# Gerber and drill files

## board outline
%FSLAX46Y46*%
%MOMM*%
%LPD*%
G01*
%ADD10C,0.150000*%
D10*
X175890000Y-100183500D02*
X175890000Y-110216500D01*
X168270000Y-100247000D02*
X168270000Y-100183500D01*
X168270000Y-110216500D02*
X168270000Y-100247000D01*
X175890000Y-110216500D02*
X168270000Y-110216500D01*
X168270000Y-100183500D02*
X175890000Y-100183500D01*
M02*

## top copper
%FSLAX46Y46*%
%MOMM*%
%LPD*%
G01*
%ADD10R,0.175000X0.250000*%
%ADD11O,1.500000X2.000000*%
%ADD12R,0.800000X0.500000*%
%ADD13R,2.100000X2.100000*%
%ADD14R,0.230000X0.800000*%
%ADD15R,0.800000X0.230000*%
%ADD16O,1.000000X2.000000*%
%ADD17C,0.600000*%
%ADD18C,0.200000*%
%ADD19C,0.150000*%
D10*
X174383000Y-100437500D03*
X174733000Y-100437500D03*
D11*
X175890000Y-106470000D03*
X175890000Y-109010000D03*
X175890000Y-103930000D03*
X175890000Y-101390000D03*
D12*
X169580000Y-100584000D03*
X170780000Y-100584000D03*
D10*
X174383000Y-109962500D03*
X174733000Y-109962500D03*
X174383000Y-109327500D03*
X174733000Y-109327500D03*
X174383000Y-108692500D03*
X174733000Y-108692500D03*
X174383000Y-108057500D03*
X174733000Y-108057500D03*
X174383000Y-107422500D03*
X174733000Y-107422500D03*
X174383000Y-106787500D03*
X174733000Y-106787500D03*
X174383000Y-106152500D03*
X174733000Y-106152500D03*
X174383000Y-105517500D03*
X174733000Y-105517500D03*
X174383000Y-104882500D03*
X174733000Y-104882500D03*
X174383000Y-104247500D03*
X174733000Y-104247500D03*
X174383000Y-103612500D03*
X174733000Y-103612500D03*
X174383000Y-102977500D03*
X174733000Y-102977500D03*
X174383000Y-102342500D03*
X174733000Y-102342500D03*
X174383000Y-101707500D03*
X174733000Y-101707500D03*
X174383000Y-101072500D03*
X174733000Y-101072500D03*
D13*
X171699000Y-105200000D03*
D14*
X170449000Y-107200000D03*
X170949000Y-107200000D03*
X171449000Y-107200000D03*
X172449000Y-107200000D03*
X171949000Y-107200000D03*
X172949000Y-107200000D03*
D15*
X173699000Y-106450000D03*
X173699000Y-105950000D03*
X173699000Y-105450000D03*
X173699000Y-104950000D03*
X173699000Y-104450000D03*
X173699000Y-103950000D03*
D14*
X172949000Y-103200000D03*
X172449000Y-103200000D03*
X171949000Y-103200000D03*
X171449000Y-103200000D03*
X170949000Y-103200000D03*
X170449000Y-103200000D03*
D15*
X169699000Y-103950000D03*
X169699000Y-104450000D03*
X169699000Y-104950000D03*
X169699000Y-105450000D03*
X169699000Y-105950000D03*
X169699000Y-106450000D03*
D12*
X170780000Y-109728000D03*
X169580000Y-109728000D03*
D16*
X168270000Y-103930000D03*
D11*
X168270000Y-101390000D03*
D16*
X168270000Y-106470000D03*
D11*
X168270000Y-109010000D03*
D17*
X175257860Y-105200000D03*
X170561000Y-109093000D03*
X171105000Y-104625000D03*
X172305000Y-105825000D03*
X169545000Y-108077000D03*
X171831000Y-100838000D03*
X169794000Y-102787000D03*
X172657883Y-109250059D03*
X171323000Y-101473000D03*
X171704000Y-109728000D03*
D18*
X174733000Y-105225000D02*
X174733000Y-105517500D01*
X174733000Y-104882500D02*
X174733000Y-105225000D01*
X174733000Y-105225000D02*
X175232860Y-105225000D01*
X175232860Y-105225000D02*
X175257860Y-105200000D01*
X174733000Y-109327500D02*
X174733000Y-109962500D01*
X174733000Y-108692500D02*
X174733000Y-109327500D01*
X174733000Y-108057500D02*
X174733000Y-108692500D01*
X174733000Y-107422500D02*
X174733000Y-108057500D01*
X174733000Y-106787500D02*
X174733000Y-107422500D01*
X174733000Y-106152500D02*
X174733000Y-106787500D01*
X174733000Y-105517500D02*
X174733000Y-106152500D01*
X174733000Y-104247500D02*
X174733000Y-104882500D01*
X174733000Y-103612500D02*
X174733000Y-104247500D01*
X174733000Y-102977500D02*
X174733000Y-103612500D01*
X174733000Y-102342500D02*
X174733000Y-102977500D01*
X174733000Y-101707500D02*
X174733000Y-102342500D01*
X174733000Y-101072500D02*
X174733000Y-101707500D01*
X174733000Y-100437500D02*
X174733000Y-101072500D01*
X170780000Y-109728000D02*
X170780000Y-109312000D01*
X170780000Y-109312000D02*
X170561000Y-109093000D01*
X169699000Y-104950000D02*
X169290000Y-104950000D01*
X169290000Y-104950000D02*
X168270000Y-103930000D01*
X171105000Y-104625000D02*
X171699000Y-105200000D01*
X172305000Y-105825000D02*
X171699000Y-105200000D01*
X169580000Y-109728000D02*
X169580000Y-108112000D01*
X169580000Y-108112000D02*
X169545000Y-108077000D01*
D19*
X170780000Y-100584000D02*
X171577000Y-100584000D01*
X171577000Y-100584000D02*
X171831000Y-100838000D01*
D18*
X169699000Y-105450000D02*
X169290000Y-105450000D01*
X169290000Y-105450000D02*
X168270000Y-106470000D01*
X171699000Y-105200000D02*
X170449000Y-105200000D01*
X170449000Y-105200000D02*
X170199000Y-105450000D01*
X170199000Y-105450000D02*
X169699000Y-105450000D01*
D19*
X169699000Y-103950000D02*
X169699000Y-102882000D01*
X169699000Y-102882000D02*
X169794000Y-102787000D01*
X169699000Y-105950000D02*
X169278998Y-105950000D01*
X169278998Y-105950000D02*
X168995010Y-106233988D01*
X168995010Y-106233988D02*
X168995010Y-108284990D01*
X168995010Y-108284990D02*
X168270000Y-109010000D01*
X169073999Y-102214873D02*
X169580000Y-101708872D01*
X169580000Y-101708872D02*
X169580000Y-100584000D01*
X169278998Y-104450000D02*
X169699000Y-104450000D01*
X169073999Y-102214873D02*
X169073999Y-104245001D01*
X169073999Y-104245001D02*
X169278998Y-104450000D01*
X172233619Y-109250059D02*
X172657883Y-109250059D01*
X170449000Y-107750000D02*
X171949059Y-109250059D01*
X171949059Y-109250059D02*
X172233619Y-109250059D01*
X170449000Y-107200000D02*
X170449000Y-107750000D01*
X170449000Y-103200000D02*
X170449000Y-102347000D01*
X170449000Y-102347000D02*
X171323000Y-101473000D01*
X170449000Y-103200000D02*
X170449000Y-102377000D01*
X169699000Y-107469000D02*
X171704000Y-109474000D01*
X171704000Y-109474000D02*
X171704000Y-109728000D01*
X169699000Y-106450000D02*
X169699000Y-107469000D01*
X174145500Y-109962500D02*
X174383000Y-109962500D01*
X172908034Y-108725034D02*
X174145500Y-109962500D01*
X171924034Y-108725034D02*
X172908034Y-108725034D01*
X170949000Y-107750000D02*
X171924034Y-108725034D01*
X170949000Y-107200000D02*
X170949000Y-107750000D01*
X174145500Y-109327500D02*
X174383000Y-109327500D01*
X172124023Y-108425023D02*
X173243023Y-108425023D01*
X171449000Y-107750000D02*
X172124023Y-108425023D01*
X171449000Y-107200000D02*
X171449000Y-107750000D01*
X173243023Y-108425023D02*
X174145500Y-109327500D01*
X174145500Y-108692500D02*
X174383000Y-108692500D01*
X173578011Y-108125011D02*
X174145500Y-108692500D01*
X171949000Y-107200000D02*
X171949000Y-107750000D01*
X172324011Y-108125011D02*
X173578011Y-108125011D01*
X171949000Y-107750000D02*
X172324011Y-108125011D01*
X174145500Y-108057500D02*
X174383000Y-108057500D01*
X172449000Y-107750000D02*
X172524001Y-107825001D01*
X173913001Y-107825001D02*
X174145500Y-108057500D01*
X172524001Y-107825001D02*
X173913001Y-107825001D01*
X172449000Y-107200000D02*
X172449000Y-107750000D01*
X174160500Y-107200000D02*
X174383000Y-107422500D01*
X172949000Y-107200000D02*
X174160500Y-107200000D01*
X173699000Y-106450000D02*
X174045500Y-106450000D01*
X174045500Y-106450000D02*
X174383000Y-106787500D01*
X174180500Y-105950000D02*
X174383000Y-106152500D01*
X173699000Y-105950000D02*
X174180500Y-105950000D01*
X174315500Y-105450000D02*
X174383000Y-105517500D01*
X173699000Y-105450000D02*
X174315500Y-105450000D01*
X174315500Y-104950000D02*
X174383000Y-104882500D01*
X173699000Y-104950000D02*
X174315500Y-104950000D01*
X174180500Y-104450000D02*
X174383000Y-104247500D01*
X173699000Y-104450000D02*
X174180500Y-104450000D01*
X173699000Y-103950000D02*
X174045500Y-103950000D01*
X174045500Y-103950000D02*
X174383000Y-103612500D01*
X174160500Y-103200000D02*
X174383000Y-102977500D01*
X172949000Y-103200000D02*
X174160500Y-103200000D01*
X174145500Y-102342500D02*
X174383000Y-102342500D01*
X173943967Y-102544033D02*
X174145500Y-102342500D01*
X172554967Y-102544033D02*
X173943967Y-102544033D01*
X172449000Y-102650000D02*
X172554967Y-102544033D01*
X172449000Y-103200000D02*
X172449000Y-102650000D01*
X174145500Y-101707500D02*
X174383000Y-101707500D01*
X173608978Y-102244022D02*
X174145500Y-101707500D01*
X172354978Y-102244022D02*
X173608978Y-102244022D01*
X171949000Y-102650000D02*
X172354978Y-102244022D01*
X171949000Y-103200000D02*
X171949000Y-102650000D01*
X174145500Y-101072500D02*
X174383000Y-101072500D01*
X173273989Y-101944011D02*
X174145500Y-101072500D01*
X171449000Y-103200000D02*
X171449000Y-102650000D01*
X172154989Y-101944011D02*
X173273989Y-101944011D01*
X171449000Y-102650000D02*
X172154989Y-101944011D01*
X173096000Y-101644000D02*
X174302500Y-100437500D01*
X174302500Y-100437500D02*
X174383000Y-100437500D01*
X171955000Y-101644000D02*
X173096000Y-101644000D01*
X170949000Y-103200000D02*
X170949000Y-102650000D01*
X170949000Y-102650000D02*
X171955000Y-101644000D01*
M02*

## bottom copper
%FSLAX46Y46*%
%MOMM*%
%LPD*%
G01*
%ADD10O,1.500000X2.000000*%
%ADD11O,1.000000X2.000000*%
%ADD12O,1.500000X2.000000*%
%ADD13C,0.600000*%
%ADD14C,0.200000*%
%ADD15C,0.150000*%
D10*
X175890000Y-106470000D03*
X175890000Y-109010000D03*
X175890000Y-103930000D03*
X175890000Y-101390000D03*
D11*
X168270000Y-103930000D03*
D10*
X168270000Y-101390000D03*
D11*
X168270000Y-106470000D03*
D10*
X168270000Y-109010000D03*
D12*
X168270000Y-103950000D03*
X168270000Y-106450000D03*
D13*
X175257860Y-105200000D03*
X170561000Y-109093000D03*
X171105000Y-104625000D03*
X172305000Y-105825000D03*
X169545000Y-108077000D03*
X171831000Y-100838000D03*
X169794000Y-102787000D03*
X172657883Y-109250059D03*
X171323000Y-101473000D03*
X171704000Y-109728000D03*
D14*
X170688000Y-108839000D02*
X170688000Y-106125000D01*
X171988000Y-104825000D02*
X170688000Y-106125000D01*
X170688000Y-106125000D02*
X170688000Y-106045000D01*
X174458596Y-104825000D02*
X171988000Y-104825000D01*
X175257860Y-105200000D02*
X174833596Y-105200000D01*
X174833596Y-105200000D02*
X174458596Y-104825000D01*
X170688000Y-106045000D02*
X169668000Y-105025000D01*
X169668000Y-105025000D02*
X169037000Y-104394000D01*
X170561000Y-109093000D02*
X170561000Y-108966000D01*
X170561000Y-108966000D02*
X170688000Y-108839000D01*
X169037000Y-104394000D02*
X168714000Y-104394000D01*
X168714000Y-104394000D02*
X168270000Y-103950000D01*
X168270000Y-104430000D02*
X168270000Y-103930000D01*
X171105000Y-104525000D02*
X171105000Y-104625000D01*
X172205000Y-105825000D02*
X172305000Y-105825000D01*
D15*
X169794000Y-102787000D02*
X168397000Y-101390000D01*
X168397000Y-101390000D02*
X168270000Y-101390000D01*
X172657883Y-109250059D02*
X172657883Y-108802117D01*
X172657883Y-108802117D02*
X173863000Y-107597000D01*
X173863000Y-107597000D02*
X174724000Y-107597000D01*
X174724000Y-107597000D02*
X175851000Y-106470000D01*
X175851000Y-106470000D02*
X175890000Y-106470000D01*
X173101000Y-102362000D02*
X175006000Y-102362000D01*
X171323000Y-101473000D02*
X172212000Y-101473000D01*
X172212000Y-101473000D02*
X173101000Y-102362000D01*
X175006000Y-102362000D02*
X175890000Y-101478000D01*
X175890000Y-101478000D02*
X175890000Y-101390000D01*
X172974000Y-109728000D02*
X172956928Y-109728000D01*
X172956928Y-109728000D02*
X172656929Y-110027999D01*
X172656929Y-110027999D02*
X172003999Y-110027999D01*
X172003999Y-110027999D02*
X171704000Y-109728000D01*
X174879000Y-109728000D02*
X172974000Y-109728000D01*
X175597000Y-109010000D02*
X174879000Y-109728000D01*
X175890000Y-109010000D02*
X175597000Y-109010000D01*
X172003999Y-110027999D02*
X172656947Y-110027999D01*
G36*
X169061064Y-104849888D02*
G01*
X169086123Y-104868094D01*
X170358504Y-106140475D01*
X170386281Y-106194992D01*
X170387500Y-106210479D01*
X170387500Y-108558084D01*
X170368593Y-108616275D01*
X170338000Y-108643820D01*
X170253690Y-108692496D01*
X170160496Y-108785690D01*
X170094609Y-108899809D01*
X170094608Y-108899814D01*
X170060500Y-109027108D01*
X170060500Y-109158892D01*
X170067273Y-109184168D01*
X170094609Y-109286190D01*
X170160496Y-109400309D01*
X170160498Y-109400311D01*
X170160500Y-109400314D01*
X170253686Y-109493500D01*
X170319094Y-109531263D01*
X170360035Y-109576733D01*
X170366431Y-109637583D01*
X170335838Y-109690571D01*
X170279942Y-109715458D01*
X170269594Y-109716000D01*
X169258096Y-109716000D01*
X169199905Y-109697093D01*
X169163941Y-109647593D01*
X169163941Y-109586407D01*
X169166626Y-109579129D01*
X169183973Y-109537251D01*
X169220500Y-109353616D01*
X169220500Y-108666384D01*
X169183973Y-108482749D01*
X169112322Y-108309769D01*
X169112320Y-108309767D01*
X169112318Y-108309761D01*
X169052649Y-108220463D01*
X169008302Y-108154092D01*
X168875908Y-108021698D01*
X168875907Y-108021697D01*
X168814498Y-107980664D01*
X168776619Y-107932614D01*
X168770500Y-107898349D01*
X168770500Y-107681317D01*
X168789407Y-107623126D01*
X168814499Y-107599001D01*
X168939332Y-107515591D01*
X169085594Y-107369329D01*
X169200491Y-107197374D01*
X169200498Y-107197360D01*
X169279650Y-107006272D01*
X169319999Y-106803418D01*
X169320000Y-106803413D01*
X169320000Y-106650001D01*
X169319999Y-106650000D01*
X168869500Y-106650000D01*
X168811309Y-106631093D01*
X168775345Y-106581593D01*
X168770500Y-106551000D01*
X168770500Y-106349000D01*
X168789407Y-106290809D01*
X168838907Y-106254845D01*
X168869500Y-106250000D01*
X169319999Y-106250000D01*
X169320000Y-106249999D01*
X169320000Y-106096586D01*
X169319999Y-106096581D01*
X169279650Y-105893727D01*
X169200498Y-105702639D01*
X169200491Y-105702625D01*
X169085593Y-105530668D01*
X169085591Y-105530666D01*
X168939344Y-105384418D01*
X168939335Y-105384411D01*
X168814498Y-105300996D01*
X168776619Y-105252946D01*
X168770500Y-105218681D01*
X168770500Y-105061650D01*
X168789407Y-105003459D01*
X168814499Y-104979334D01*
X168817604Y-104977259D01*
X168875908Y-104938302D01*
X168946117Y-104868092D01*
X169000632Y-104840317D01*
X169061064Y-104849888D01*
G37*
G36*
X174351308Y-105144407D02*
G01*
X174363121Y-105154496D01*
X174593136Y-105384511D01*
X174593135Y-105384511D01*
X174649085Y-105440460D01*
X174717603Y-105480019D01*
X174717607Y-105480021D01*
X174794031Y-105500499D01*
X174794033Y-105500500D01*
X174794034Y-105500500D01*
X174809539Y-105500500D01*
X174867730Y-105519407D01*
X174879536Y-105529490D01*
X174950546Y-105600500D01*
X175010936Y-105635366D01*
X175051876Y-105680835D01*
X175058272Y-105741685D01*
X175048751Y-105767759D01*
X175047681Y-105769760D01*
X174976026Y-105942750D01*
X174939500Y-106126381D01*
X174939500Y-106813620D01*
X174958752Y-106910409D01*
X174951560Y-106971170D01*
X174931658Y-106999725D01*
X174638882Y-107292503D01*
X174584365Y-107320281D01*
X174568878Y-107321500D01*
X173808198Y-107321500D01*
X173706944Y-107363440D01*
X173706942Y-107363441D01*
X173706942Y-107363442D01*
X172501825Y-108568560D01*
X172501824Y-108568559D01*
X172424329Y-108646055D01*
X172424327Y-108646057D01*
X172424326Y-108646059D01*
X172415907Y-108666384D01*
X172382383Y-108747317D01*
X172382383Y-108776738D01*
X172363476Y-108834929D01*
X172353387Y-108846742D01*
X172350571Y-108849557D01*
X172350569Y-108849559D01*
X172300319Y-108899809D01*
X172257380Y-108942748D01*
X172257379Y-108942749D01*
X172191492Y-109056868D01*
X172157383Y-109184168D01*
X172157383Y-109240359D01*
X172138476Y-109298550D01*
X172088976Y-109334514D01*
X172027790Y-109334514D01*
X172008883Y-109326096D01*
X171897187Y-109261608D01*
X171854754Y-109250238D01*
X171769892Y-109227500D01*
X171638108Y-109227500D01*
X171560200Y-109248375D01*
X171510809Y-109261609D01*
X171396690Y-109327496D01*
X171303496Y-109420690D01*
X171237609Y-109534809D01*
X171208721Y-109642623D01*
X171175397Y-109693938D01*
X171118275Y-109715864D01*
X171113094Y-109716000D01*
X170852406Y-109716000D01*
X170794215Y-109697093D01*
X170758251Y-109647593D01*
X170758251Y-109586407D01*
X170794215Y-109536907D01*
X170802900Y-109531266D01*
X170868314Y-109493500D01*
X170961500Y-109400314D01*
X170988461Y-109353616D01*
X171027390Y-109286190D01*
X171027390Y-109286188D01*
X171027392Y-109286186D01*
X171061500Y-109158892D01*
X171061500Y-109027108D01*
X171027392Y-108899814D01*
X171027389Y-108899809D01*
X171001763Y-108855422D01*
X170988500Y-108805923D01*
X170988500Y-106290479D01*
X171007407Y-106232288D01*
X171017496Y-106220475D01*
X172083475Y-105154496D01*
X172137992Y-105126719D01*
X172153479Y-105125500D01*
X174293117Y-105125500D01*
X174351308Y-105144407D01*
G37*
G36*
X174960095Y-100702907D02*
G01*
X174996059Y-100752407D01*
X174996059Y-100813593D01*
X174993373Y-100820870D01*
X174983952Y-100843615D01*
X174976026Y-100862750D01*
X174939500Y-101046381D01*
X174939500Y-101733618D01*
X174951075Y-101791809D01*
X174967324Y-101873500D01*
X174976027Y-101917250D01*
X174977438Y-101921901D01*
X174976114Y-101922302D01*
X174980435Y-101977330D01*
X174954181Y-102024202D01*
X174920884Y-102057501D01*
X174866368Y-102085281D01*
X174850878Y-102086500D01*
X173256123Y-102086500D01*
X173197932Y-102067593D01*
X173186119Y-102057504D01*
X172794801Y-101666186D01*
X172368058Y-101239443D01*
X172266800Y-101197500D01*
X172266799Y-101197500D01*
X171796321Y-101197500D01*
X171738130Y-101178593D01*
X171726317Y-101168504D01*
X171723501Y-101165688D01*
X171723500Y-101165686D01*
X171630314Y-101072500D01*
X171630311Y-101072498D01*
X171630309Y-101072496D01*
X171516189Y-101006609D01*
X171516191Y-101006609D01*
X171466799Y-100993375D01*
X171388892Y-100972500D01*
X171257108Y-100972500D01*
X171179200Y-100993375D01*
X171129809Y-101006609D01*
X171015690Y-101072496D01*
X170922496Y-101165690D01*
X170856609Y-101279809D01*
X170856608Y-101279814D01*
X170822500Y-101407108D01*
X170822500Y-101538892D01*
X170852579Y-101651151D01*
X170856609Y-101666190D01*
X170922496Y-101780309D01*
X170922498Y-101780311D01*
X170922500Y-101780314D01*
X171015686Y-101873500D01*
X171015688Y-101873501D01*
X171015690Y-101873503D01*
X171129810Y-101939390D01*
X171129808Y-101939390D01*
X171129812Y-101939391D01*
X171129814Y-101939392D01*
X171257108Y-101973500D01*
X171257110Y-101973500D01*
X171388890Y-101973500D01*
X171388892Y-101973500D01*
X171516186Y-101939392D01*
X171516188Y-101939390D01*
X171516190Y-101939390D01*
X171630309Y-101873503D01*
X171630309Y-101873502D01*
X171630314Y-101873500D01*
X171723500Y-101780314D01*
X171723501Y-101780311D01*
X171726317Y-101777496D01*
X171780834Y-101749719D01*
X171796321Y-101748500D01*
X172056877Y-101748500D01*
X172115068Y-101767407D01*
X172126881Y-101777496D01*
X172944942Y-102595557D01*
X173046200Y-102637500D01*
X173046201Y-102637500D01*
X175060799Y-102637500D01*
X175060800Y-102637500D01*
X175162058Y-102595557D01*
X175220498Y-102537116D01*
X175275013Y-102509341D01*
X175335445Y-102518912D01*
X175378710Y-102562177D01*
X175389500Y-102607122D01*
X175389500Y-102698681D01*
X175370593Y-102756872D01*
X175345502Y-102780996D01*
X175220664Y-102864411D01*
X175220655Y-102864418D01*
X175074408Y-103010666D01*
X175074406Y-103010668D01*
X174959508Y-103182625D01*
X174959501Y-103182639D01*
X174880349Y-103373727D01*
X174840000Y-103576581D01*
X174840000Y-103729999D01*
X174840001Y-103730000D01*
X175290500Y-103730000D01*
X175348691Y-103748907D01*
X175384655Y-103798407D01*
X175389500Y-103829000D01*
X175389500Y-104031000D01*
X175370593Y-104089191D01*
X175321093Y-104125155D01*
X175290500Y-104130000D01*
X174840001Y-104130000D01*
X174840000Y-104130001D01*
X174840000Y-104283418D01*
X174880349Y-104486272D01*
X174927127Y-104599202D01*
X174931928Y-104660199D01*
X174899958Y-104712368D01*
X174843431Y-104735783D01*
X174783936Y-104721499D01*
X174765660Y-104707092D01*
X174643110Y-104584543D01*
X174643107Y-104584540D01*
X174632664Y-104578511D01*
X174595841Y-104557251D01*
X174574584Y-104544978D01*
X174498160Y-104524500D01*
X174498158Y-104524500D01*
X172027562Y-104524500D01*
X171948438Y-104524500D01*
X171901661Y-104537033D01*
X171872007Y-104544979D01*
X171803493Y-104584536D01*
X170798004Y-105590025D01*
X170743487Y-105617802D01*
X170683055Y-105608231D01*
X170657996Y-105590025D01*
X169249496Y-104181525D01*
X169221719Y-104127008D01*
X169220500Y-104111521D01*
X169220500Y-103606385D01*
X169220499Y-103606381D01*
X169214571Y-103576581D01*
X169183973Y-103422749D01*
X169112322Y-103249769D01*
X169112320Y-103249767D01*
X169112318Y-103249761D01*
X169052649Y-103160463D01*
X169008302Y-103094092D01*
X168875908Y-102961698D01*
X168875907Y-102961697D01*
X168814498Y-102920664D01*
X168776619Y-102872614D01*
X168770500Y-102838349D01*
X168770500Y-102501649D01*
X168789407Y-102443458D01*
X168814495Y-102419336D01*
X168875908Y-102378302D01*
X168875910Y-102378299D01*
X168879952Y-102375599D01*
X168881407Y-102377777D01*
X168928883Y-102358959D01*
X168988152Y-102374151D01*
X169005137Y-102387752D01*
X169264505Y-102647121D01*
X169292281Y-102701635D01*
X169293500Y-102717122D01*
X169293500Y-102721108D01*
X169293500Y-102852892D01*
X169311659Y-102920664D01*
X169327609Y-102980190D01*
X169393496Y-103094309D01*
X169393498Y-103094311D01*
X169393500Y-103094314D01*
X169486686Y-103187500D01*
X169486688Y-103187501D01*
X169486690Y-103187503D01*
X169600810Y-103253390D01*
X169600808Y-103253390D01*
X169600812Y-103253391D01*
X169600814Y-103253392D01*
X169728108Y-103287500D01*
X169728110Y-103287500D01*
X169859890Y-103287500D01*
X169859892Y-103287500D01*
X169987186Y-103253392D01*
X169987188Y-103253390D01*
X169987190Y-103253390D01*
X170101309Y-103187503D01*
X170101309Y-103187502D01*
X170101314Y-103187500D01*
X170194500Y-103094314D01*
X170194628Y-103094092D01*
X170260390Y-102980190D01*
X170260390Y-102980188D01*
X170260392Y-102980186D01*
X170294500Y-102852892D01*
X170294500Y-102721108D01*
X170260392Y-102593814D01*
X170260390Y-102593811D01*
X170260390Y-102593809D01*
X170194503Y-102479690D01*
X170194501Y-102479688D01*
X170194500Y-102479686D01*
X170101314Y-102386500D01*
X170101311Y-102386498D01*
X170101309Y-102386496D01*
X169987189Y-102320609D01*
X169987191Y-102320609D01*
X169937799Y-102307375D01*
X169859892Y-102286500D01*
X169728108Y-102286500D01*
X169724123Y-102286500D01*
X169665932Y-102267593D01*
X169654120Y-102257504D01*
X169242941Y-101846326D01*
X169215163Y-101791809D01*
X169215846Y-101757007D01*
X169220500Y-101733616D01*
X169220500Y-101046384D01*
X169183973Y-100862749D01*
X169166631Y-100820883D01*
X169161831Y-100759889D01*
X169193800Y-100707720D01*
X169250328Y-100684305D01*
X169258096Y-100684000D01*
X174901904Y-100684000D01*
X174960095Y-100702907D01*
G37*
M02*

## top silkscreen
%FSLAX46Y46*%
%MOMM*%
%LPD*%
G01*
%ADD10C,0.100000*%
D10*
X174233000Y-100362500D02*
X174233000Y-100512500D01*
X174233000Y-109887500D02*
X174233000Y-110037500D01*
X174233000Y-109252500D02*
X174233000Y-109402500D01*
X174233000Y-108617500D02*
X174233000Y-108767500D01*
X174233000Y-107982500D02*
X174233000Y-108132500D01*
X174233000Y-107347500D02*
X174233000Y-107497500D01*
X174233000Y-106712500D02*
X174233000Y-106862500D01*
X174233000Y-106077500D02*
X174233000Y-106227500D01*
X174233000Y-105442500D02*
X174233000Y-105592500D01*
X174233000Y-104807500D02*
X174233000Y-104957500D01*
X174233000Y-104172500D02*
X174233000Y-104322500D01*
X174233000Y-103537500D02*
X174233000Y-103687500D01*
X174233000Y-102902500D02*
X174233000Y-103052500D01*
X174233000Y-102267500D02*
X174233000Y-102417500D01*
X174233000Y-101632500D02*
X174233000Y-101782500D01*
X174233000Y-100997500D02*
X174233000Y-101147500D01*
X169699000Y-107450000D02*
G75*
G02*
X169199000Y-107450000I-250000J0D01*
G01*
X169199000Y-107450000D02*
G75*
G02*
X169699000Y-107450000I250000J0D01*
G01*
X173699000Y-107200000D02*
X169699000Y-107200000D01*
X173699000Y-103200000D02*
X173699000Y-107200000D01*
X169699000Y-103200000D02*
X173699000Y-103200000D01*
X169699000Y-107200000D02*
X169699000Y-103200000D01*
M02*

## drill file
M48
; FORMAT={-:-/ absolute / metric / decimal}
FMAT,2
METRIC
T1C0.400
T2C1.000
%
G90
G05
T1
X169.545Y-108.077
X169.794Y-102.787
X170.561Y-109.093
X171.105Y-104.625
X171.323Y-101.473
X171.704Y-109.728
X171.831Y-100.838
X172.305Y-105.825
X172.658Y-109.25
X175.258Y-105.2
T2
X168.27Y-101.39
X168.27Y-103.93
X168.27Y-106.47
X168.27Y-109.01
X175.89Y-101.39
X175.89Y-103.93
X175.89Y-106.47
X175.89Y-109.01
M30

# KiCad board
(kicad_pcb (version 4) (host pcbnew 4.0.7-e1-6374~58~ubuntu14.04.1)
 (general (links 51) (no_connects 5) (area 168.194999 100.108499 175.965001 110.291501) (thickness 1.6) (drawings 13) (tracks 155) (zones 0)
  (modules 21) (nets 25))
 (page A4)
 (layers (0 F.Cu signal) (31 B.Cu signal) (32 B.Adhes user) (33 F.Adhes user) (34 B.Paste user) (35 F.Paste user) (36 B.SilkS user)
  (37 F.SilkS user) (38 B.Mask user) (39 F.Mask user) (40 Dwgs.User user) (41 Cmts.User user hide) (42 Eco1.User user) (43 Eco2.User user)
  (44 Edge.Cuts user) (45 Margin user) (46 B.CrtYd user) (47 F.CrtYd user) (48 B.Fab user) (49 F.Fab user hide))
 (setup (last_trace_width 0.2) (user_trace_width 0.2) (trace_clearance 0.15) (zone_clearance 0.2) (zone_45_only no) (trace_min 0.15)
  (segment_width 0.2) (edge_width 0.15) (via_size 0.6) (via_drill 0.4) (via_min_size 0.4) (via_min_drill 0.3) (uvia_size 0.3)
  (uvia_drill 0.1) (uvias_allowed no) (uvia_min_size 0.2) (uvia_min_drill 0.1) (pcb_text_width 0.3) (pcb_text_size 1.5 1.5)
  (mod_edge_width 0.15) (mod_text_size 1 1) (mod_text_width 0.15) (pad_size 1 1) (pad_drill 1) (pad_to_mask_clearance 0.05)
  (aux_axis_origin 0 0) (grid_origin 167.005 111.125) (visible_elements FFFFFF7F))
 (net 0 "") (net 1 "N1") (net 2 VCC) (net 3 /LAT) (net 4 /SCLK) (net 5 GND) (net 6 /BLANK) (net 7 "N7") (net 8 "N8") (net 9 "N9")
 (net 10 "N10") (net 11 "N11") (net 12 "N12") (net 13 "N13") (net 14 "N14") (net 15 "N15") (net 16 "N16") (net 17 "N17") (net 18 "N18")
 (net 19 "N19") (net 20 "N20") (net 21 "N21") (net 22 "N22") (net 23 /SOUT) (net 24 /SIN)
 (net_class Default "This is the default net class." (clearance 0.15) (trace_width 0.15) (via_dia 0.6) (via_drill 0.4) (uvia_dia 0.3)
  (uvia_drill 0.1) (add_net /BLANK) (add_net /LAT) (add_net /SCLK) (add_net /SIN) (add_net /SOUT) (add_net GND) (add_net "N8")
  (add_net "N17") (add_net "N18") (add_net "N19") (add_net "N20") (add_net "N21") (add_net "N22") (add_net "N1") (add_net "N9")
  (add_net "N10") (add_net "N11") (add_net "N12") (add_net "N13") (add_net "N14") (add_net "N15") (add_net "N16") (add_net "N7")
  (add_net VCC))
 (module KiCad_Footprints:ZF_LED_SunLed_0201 (layer F.Cu) (at 174.558 100.4375)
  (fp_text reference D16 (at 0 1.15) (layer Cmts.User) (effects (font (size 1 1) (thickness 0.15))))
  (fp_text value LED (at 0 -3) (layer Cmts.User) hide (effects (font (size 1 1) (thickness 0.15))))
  (fp_line (start -0.325 -0.075) (end -0.325 0.075) (layer F.SilkS) (width 0.1))
  (pad 1 smd rect (at -0.175 0) (size 0.175 0.25) (layers F.Cu F.Paste F.Mask) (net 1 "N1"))
  (pad 2 smd rect (at 0.175 0) (size 0.175 0.25) (layers F.Cu F.Paste F.Mask) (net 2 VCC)))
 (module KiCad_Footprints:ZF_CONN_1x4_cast (layer F.Cu) (at 175.89 105.2 90)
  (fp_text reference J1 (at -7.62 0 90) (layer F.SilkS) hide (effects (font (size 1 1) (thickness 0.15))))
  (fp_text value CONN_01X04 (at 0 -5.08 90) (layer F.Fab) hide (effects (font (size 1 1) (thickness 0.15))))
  (pad 2 thru_hole oval (at -1.27 0 90) (size 2 1.5) (drill 1) (layers *.Cu *.Mask) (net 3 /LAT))
  (pad 1 thru_hole oval (at -3.81 0 90) (size 2 1.5) (drill 1) (layers *.Cu *.Mask) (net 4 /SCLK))
  (pad 3 thru_hole oval (at 1.27 0 90) (size 2 1.5) (drill 1) (layers *.Cu *.Mask) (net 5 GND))
  (pad 4 thru_hole oval (at 3.81 0 90) (size 2 1.5) (drill 1) (layers *.Cu *.Mask) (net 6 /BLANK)))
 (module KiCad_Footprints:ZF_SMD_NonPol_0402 (layer F.Cu) (at 170.18 100.584)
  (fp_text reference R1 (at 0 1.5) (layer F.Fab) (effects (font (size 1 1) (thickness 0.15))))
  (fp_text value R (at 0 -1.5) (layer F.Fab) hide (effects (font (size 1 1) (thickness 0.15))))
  (pad 1 smd rect (at -0.6 0) (size 0.8 0.5) (layers F.Cu F.Paste F.Mask) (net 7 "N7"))
  (pad 2 smd rect (at 0.6 0) (size 0.8 0.5) (layers F.Cu F.Paste F.Mask) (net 5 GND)))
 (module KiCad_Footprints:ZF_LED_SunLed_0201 (layer F.Cu) (at 174.558 109.9625)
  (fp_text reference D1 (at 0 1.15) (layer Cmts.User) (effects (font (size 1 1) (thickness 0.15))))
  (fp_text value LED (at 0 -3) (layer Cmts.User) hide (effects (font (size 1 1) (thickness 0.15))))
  (fp_line (start -0.325 -0.075) (end -0.325 0.075) (layer F.SilkS) (width 0.1))
  (pad 1 smd rect (at -0.175 0) (size 0.175 0.25) (layers F.Cu F.Paste F.Mask) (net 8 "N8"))
  (pad 2 smd rect (at 0.175 0) (size 0.175 0.25) (layers F.Cu F.Paste F.Mask) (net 2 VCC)))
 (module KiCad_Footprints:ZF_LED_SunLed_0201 (layer F.Cu) (at 174.558 109.3275)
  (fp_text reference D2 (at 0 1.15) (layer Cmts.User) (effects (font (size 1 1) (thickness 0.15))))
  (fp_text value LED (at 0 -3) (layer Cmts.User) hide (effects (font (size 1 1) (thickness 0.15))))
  (fp_line (start -0.325 -0.075) (end -0.325 0.075) (layer F.SilkS) (width 0.1))
  (pad 1 smd rect (at -0.175 0) (size 0.175 0.25) (layers F.Cu F.Paste F.Mask) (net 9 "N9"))
  (pad 2 smd rect (at 0.175 0) (size 0.175 0.25) (layers F.Cu F.Paste F.Mask) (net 2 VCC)))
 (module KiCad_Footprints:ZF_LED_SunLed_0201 (layer F.Cu) (at 174.558 108.6925)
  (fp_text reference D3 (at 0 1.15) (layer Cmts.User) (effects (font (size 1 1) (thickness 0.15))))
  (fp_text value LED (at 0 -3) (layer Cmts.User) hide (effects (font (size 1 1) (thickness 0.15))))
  (fp_line (start -0.325 -0.075) (end -0.325 0.075) (layer F.SilkS) (width 0.1))
  (pad 1 smd rect (at -0.175 0) (size 0.175 0.25) (layers F.Cu F.Paste F.Mask) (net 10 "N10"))
  (pad 2 smd rect (at 0.175 0) (size 0.175 0.25) (layers F.Cu F.Paste F.Mask) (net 2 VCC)))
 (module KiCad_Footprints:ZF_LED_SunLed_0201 (layer F.Cu) (at 174.558 108.0575)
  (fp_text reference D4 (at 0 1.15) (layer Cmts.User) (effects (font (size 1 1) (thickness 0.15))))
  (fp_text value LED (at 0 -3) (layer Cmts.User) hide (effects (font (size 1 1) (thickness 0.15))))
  (fp_line (start -0.325 -0.075) (end -0.325 0.075) (layer F.SilkS) (width 0.1))
  (pad 1 smd rect (at -0.175 0) (size 0.175 0.25) (layers F.Cu F.Paste F.Mask) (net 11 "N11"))
  (pad 2 smd rect (at 0.175 0) (size 0.175 0.25) (layers F.Cu F.Paste F.Mask) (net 2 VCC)))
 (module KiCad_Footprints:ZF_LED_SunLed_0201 (layer F.Cu) (at 174.558 107.4225)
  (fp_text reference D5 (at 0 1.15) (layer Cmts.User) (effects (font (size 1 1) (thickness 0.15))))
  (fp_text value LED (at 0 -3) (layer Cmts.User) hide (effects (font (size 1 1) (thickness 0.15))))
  (fp_line (start -0.325 -0.075) (end -0.325 0.075) (layer F.SilkS) (width 0.1))
  (pad 1 smd rect (at -0.175 0) (size 0.175 0.25) (layers F.Cu F.Paste F.Mask) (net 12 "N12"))
  (pad 2 smd rect (at 0.175 0) (size 0.175 0.25) (layers F.Cu F.Paste F.Mask) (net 2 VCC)))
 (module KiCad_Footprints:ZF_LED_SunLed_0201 (layer F.Cu) (at 174.558 106.7875)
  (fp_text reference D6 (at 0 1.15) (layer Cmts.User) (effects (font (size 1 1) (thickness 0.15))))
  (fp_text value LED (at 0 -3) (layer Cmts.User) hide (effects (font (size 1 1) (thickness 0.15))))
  (fp_line (start -0.325 -0.075) (end -0.325 0.075) (layer F.SilkS) (width 0.1))
  (pad 1 smd rect (at -0.175 0) (size 0.175 0.25) (layers F.Cu F.Paste F.Mask) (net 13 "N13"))
  (pad 2 smd rect (at 0.175 0) (size 0.175 0.25) (layers F.Cu F.Paste F.Mask) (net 2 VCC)))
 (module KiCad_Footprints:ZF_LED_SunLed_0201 (layer F.Cu) (at 174.558 106.1525)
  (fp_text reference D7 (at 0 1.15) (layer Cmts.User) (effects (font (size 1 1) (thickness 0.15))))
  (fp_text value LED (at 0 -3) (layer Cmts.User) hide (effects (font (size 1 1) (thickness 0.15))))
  (fp_line (start -0.325 -0.075) (end -0.325 0.075) (layer F.SilkS) (width 0.1))
  (pad 1 smd rect (at -0.175 0) (size 0.175 0.25) (layers F.Cu F.Paste F.Mask) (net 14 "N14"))
  (pad 2 smd rect (at 0.175 0) (size 0.175 0.25) (layers F.Cu F.Paste F.Mask) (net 2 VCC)))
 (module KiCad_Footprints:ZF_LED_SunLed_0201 (layer F.Cu) (at 174.558 105.5175)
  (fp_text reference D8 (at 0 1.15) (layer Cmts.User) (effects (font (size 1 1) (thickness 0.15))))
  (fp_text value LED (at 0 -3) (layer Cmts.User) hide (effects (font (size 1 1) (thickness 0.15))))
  (fp_line (start -0.325 -0.075) (end -0.325 0.075) (layer F.SilkS) (width 0.1))
  (pad 1 smd rect (at -0.175 0) (size 0.175 0.25) (layers F.Cu F.Paste F.Mask) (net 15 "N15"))
  (pad 2 smd rect (at 0.175 0) (size 0.175 0.25) (layers F.Cu F.Paste F.Mask) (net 2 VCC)))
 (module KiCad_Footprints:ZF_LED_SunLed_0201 (layer F.Cu) (at 174.558 104.8825)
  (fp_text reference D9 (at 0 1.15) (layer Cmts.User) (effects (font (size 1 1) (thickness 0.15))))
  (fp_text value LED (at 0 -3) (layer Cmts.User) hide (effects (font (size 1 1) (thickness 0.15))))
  (fp_line (start -0.325 -0.075) (end -0.325 0.075) (layer F.SilkS) (width 0.1))
  (pad 1 smd rect (at -0.175 0) (size 0.175 0.25) (layers F.Cu F.Paste F.Mask) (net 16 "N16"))
  (pad 2 smd rect (at 0.175 0) (size 0.175 0.25) (layers F.Cu F.Paste F.Mask) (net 2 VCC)))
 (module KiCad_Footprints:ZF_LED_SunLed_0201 (layer F.Cu) (at 174.558 104.2475)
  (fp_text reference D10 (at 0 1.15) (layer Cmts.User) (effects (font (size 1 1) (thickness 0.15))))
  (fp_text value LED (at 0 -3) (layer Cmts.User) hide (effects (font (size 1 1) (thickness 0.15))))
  (fp_line (start -0.325 -0.075) (end -0.325 0.075) (layer F.SilkS) (width 0.1))
  (pad 1 smd rect (at -0.175 0) (size 0.175 0.25) (layers F.Cu F.Paste F.Mask) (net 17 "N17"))
  (pad 2 smd rect (at 0.175 0) (size 0.175 0.25) (layers F.Cu F.Paste F.Mask) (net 2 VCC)))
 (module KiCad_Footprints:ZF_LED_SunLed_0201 (layer F.Cu) (at 174.558 103.6125)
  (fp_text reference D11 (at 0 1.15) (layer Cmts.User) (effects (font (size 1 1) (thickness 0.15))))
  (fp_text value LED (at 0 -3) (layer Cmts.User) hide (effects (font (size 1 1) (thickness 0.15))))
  (fp_line (start -0.325 -0.075) (end -0.325 0.075) (layer F.SilkS) (width 0.1))
  (pad 1 smd rect (at -0.175 0) (size 0.175 0.25) (layers F.Cu F.Paste F.Mask) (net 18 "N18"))
  (pad 2 smd rect (at 0.175 0) (size 0.175 0.25) (layers F.Cu F.Paste F.Mask) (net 2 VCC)))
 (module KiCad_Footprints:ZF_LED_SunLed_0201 (layer F.Cu) (at 174.558 102.9775)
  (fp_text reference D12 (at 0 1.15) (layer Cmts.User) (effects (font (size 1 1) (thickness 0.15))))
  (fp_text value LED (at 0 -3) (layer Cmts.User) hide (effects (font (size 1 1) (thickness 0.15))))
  (fp_line (start -0.325 -0.075) (end -0.325 0.075) (layer F.SilkS) (width 0.1))
  (pad 1 smd rect (at -0.175 0) (size 0.175 0.25) (layers F.Cu F.Paste F.Mask) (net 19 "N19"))
  (pad 2 smd rect (at 0.175 0) (size 0.175 0.25) (layers F.Cu F.Paste F.Mask) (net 2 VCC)))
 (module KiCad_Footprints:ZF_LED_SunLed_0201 (layer F.Cu) (at 174.558 102.3425)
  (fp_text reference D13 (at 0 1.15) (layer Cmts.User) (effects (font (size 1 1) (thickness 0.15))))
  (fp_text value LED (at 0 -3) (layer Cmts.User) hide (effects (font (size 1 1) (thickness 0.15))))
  (fp_line (start -0.325 -0.075) (end -0.325 0.075) (layer F.SilkS) (width 0.1))
  (pad 1 smd rect (at -0.175 0) (size 0.175 0.25) (layers F.Cu F.Paste F.Mask) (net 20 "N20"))
  (pad 2 smd rect (at 0.175 0) (size 0.175 0.25) (layers F.Cu F.Paste F.Mask) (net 2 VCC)))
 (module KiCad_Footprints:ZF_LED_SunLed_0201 (layer F.Cu) (at 174.558 101.7075)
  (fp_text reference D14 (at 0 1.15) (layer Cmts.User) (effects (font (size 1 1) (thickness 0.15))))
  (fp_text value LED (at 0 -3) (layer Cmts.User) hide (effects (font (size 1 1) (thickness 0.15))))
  (fp_line (start -0.325 -0.075) (end -0.325 0.075) (layer F.SilkS) (width 0.1))
  (pad 1 smd rect (at -0.175 0) (size 0.175 0.25) (layers F.Cu F.Paste F.Mask) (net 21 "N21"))
  (pad 2 smd rect (at 0.175 0) (size 0.175 0.25) (layers F.Cu F.Paste F.Mask) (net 2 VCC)))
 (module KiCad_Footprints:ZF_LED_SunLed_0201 (layer F.Cu) (at 174.558 101.0725)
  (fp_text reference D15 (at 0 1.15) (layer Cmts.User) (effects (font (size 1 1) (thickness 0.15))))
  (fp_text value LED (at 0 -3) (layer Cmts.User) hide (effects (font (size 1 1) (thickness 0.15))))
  (fp_line (start -0.325 -0.075) (end -0.325 0.075) (layer F.SilkS) (width 0.1))
  (pad 1 smd rect (at -0.175 0) (size 0.175 0.25) (layers F.Cu F.Paste F.Mask) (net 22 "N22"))
  (pad 2 smd rect (at 0.175 0) (size 0.175 0.25) (layers F.Cu F.Paste F.Mask) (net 2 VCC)))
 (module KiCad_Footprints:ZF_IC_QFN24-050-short (layer F.Cu) (at 171.699 105.2 90)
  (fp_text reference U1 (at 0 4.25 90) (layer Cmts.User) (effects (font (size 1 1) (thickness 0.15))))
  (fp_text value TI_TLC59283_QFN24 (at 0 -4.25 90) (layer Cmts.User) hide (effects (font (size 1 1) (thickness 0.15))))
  (fp_circle (center -2.25 -2.25) (end -2.25 -2) (layer F.SilkS) (width 0.1))
  (fp_line (start -2 2) (end -2 -2) (layer F.SilkS) (width 0.1)) (fp_line (start 2 2) (end -2 2) (layer F.SilkS) (width 0.1))
  (fp_line (start 2 -2) (end 2 2) (layer F.SilkS) (width 0.1))
  (fp_line (start -2 -2) (end 2 -2) (layer F.SilkS) (width 0.1))
  (pad 22 smd rect (at 0 0 90) (size 2.1 2.1) (layers F.Cu F.Mask) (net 5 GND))
  (pad 1 smd rect (at -2 -1.25 90) (size 0.8 0.23) (layers F.Cu F.Paste F.Mask) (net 3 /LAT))
  (pad 22 smd rect (at -0.6 -0.6 90) (size 0.8 0.8) (layers F.Paste) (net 5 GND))
  (pad 22 smd rect (at 0.6 -0.6 90) (size 0.8 0.8) (layers F.Paste) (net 5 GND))
  (pad 22 smd rect (at 0.6 0.6 90) (size 0.8 0.8) (layers F.Paste) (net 5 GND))
  (pad 22 smd rect (at -0.6 0.6 90) (size 0.8 0.8) (layers F.Paste) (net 5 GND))
  (pad 2 smd rect (at -2 -0.75 90) (size 0.8 0.23) (layers F.Cu F.Paste F.Mask) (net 8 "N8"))
  (pad 3 smd rect (at -2 -0.25 90) (size 0.8 0.23) (layers F.Cu F.Paste F.Mask) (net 9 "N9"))
  (pad 5 smd rect (at -2 0.75 90) (size 0.8 0.23) (layers F.Cu F.Paste F.Mask) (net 11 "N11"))
  (pad 4 smd rect (at -2 0.25 90) (size 0.8 0.23) (layers F.Cu F.Paste F.Mask) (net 10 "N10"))
  (pad 6 smd rect (at -2 1.25 90) (size 0.8 0.23) (layers F.Cu F.Paste F.Mask) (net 12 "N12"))
  (pad 7 smd rect (at -1.25 2 180) (size 0.8 0.23) (layers F.Cu F.Paste F.Mask) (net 13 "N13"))
  (pad 8 smd rect (at -0.75 2 180) (size 0.8 0.23) (layers F.Cu F.Paste F.Mask) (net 14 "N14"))
  (pad 9 smd rect (at -0.25 2 180) (size 0.8 0.23) (layers F.Cu F.Paste F.Mask) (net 15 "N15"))
  (pad 10 smd rect (at 0.25 2 180) (size 0.8 0.23) (layers F.Cu F.Paste F.Mask) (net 16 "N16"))
  (pad 11 smd rect (at 0.75 2 180) (size 0.8 0.23) (layers F.Cu F.Paste F.Mask) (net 17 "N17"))
  (pad 12 smd rect (at 1.25 2 180) (size 0.8 0.23) (layers F.Cu F.Paste F.Mask) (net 18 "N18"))
  (pad 13 smd rect (at 2 1.25 90) (size 0.8 0.23) (layers F.Cu F.Paste F.Mask) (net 19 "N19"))
  (pad 14 smd rect (at 2 0.75 90) (size 0.8 0.23) (layers F.Cu F.Paste F.Mask) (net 20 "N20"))
  (pad 15 smd rect (at 2 0.25 90) (size 0.8 0.23) (layers F.Cu F.Paste F.Mask) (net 21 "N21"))
  (pad 16 smd rect (at 2 -0.25 90) (size 0.8 0.23) (layers F.Cu F.Paste F.Mask) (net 22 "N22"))
  (pad 17 smd rect (at 2 -0.75 90) (size 0.8 0.23) (layers F.Cu F.Paste F.Mask) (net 1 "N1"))
  (pad 18 smd rect (at 2 -1.25 90) (size 0.8 0.23) (layers F.Cu F.Paste F.Mask) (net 6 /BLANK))
  (pad 19 smd rect (at 1.25 -2 180) (size 0.8 0.23) (layers F.Cu F.Paste F.Mask) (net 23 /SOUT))
  (pad 20 smd rect (at 0.75 -2 180) (size 0.8 0.23) (layers F.Cu F.Paste F.Mask) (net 7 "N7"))
  (pad 21 smd rect (at 0.25 -2 180) (size 0.8 0.23) (layers F.Cu F.Paste F.Mask) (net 2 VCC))
  (pad 22 smd rect (at -0.25 -2 180) (size 0.8 0.23) (layers F.Cu F.Paste F.Mask) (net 5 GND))
  (pad 23 smd rect (at -0.75 -2) (size 0.8 0.23) (layers F.Cu F.Paste F.Mask) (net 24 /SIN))
  (pad 24 smd rect (at -1.25 -2 180) (size 0.8 0.23) (layers F.Cu F.Paste F.Mask) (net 4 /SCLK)))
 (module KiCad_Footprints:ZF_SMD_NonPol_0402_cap (layer F.Cu) (at 170.18 109.728 180)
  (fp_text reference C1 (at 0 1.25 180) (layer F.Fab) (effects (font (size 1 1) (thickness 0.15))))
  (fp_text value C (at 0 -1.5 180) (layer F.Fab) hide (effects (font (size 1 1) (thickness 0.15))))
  (pad 1 smd rect (at -0.6 0 180) (size 0.8 0.5) (layers F.Cu F.Paste F.Mask) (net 2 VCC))
  (pad 2 smd rect (at 0.6 0 180) (size 0.8 0.5) (layers F.Cu F.Paste F.Mask) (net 5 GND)))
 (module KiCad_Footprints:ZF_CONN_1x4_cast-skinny (layer F.Cu) (at 168.27 105.2 270)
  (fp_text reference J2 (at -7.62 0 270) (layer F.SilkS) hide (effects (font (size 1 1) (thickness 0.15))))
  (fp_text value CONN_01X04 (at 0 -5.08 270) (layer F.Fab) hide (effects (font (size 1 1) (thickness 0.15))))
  (pad 2 thru_hole oval (at -1.27 0 270) (size 2 1) (drill 1) (layers *.Cu *.Mask) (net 2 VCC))
  (pad 1 thru_hole oval (at -3.81 0 270) (size 2 1.5) (drill 1) (layers *.Cu *.Mask) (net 23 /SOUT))
  (pad 3 thru_hole oval (at 1.27 0 270) (size 2 1) (drill 1) (layers *.Cu *.Mask) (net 5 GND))
  (pad 4 thru_hole oval (at 3.81 0 270) (size 2 1.5) (drill 1) (layers *.Cu *.Mask) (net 24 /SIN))
  (pad 2 smd oval (at -1.25 0 270) (size 2 1.5) (layers B.Cu B.Mask) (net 2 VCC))
  (pad 3 smd oval (at 1.25 0 270) (size 2 1.5) (layers B.Cu B.Mask) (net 5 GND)))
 (gr_line (start 175.89 100.1835) (end 175.89 110.2165) (layer Edge.Cuts) (width 0.15))
 (gr_line (start 168.27 100.247) (end 168.27 100.1835) (layer Edge.Cuts) (width 0.15))
 (gr_line (start 168.27 110.2165) (end 168.27 100.247) (layer Edge.Cuts) (width 0.15))
 (gr_line (start 175.89 110.2165) (end 168.27 110.2165) (layer Edge.Cuts) (width 0.15))
 (gr_line (start 168.27 100.1835) (end 175.89 100.1835) (layer Edge.Cuts) (width 0.15))
 (segment (start 170.688 108.839) (end 170.688 106.125) (width 0.2) (layer B.Cu) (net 2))
 (segment (start 171.988 104.825) (end 170.688 106.125) (width 0.2) (layer B.Cu) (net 2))
 (segment (start 170.688 106.125) (end 170.688 106.045) (width 0.2) (layer B.Cu) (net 2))
 (segment (start 174.458596 104.825) (end 171.988 104.825) (width 0.2) (layer B.Cu) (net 2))
 (segment (start 175.25786 105.2) (end 174.833596 105.2) (width 0.2) (layer B.Cu) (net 2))
 (segment (start 174.833596 105.2) (end 174.458596 104.825) (width 0.2) (layer B.Cu) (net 2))
 (segment (start 170.688 106.045) (end 169.668 105.025) (width 0.2) (layer B.Cu) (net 2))
 (segment (start 169.668 105.025) (end 169.037 104.394) (width 0.2) (layer B.Cu) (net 2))
 (segment (start 174.733 105.225) (end 174.733 105.5175) (width 0.2) (layer F.Cu) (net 2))
 (segment (start 174.733 104.8825) (end 174.733 105.225) (width 0.2) (layer F.Cu) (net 2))
 (segment (start 174.733 105.225) (end 175.23286 105.225) (width 0.2) (layer F.Cu) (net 2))
 (segment (start 175.23286 105.225) (end 175.25786 105.2) (width 0.2) (layer F.Cu) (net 2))
 (via (at 175.25786 105.2) (size 0.6) (drill 0.4) (layers F.Cu B.Cu) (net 2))
 (segment (start 174.733 109.3275) (end 174.733 109.9625) (width 0.2) (layer F.Cu) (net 2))
 (segment (start 174.733 108.6925) (end 174.733 109.3275) (width 0.2) (layer F.Cu) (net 2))
 (segment (start 174.733 108.0575) (end 174.733 108.6925) (width 0.2) (layer F.Cu) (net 2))
 (segment (start 174.733 107.4225) (end 174.733 108.0575) (width 0.2) (layer F.Cu) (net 2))
 (segment (start 174.733 106.7875) (end 174.733 107.4225) (width 0.2) (layer F.Cu) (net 2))
 (segment (start 174.733 106.1525) (end 174.733 106.7875) (width 0.2) (layer F.Cu) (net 2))
 (segment (start 174.733 105.5175) (end 174.733 106.1525) (width 0.2) (layer F.Cu) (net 2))
 (segment (start 174.733 104.2475) (end 174.733 104.8825) (width 0.2) (layer F.Cu) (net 2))
 (segment (start 174.733 103.6125) (end 174.733 104.2475) (width 0.2) (layer F.Cu) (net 2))
 (segment (start 174.733 102.9775) (end 174.733 103.6125) (width 0.2) (layer F.Cu) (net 2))
 (segment (start 174.733 102.3425) (end 174.733 102.9775) (width 0.2) (layer F.Cu) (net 2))
 (segment (start 174.733 101.7075) (end 174.733 102.3425) (width 0.2) (layer F.Cu) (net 2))
 (segment (start 174.733 101.0725) (end 174.733 101.7075) (width 0.2) (layer F.Cu) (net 2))
 (segment (start 174.733 100.4375) (end 174.733 101.0725) (width 0.2) (layer F.Cu) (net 2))
 (segment (start 170.561 109.093) (end 170.561 108.966) (width 0.2) (layer B.Cu) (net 2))
 (segment (start 170.561 108.966) (end 170.688 108.839) (width 0.2) (layer B.Cu) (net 2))
 (segment (start 169.037 104.394) (end 168.714 104.394) (width 0.2) (layer B.Cu) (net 2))
 (segment (start 168.714 104.394) (end 168.27 103.95) (width 0.2) (layer B.Cu) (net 2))
 (segment (start 168.27 104.43) (end 168.27 103.93) (width 0.2) (layer B.Cu) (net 2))
 (segment (start 170.78 109.728) (end 170.78 109.312) (width 0.2) (layer F.Cu) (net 2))
 (segment (start 170.78 109.312) (end 170.561 109.093) (width 0.2) (layer F.Cu) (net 2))
 (via (at 170.561 109.093) (size 0.6) (drill 0.4) (layers F.Cu B.Cu) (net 2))
 (segment (start 169.699 104.95) (end 169.29 104.95) (width 0.2) (layer F.Cu) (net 2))
 (segment (start 169.29 104.95) (end 168.27 103.93) (width 0.2) (layer F.Cu) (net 2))
 (segment (start 171.105 104.525) (end 171.105 104.625) (width 0.2) (layer B.Cu) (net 5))
 (segment (start 171.105 104.625) (end 171.699 105.2) (width 0.2) (layer F.Cu) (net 5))
 (via (at 171.105 104.625) (size 0.6) (drill 0.4) (layers F.Cu B.Cu) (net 5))
 (segment (start 172.205 105.825) (end 172.305 105.825) (width 0.2) (layer B.Cu) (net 5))
 (segment (start 172.305 105.825) (end 171.699 105.2) (width 0.2) (layer F.Cu) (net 5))
 (via (at 172.305 105.825) (size 0.6) (drill 0.4) (layers F.Cu B.Cu) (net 5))
 (segment (start 169.58 109.728) (end 169.58 108.112) (width 0.2) (layer F.Cu) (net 5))
 (segment (start 169.58 108.112) (end 169.545 108.077) (width 0.2) (layer F.Cu) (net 5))
 (via (at 169.545 108.077) (size 0.6) (drill 0.4) (layers F.Cu B.Cu) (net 5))
 (segment (start 170.78 100.584) (end 171.577 100.584) (width 0.15) (layer F.Cu) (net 5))
 (segment (start 171.577 100.584) (end 171.831 100.838) (width 0.15) (layer F.Cu) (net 5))
 (via (at 171.831 100.838) (size 0.6) (drill 0.4) (layers F.Cu B.Cu) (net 5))
 (segment (start 169.699 105.45) (end 169.29 105.45) (width 0.2) (layer F.Cu) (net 5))
 (segment (start 169.29 105.45) (end 168.27 106.47) (width 0.2) (layer F.Cu) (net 5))
 (segment (start 171.699 105.2) (end 170.449 105.2) (width 0.2) (layer F.Cu) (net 5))
 (segment (start 170.449 105.2) (end 170.199 105.45) (width 0.2) (layer F.Cu) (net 5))
 (segment (start 170.199 105.45) (end 169.699 105.45) (width 0.2) (layer F.Cu) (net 5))
 (segment (start 169.794 102.787) (end 168.397 101.39) (width 0.15) (layer B.Cu) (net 23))
 (segment (start 168.397 101.39) (end 168.27 101.39) (width 0.15) (layer B.Cu) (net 23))
 (segment (start 169.699 103.95) (end 169.699 102.882) (width 0.15) (layer F.Cu) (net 23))
 (segment (start 169.699 102.882) (end 169.794 102.787) (width 0.15) (layer F.Cu) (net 23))
 (via (at 169.794 102.787) (size 0.6) (drill 0.4) (layers F.Cu B.Cu) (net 23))
 (segment (start 169.699 105.95) (end 169.278998 105.95) (width 0.15) (layer F.Cu) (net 24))
 (segment (start 169.278998 105.95) (end 168.99501 106.233988) (width 0.15) (layer F.Cu) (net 24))
 (segment (start 168.99501 106.233988) (end 168.99501 108.28499) (width 0.15) (layer F.Cu) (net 24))
 (segment (start 168.99501 108.28499) (end 168.27 109.01) (width 0.15) (layer F.Cu) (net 24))
 (segment (start 169.073999 102.214873) (end 169.58 101.708872) (width 0.15) (layer F.Cu) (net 7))
 (segment (start 169.58 101.708872) (end 169.58 100.584) (width 0.15) (layer F.Cu) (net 7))
 (segment (start 169.278998 104.45) (end 169.699 104.45) (width 0.15) (layer F.Cu) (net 7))
 (segment (start 169.073999 102.214873) (end 169.073999 104.245001) (width 0.15) (layer F.Cu) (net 7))
 (segment (start 169.073999 104.245001) (end 169.278998 104.45) (width 0.15) (layer F.Cu) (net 7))
 (segment (start 172.657883 109.250059) (end 172.657883 108.802117) (width 0.15) (layer B.Cu) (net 3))
 (segment (start 172.657883 108.802117) (end 173.863 107.597) (width 0.15) (layer B.Cu) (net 3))
 (segment (start 173.863 107.597) (end 174.724 107.597) (width 0.15) (layer B.Cu) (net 3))
 (segment (start 174.724 107.597) (end 175.851 106.47) (width 0.15) (layer B.Cu) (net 3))
 (segment (start 175.851 106.47) (end 175.89 106.47) (width 0.15) (layer B.Cu) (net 3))
 (segment (start 172.233619 109.250059) (end 172.657883 109.250059) (width 0.15) (layer F.Cu) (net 3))
 (segment (start 170.449 107.75) (end 171.949059 109.250059) (width 0.15) (layer F.Cu) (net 3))
 (segment (start 171.949059 109.250059) (end 172.233619 109.250059) (width 0.15) (layer F.Cu) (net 3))
 (segment (start 170.449 107.2) (end 170.449 107.75) (width 0.15) (layer F.Cu) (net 3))
 (via (at 172.657883 109.250059) (size 0.6) (drill 0.4) (layers F.Cu B.Cu) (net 3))
 (segment (start 173.101 102.362) (end 175.006 102.362) (width 0.15) (layer B.Cu) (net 6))
 (segment (start 171.323 101.473) (end 172.212 101.473) (width 0.15) (layer B.Cu) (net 6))
 (segment (start 172.212 101.473) (end 173.101 102.362) (width 0.15) (layer B.Cu) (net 6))
 (segment (start 170.449 103.2) (end 170.449 102.347) (width 0.15) (layer F.Cu) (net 6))
 (via (at 171.323 101.473) (size 0.6) (drill 0.4) (layers F.Cu B.Cu) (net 6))
 (segment (start 170.449 102.347) (end 171.323 101.473) (width 0.15) (layer F.Cu) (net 6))
 (segment (start 175.006 102.362) (end 175.89 101.478) (width 0.15) (layer B.Cu) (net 6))
 (segment (start 175.89 101.478) (end 175.89 101.39) (width 0.15) (layer B.Cu) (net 6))
 (segment (start 170.449 103.2) (end 170.449 102.377) (width 0.15) (layer F.Cu) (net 6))
 (segment (start 172.974 109.728) (end 172.956928 109.728) (width 0.15) (layer B.Cu) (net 4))
 (segment (start 172.956928 109.728) (end 172.656929 110.027999) (width 0.15) (layer B.Cu) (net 4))
 (segment (start 172.656929 110.027999) (end 172.003999 110.027999) (width 0.15) (layer B.Cu) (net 4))
 (segment (start 172.003999 110.027999) (end 171.704 109.728) (width 0.15) (layer B.Cu) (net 4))
 (segment (start 174.879 109.728) (end 172.974 109.728) (width 0.15) (layer B.Cu) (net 4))
 (segment (start 175.597 109.01) (end 174.879 109.728) (width 0.15) (layer B.Cu) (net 4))
 (segment (start 175.89 109.01) (end 175.597 109.01) (width 0.15) (layer B.Cu) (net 4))
 (segment (start 172.003999 110.027999) (end 172.656947 110.027999) (width 0.15) (layer B.Cu) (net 4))
 (segment (start 169.699 107.469) (end 171.704 109.474) (width 0.15) (layer F.Cu) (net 4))
 (segment (start 171.704 109.474) (end 171.704 109.728) (width 0.15) (layer F.Cu) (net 4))
 (via (at 171.704 109.728) (size 0.6) (drill 0.4) (layers F.Cu B.Cu) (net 4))
 (segment (start 169.699 106.45) (end 169.699 107.469) (width 0.15) (layer F.Cu) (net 4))
 (segment (start 174.1455 109.9625) (end 174.383 109.9625) (width 0.15) (layer F.Cu) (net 8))
 (segment (start 172.908034 108.725034) (end 174.1455 109.9625) (width 0.15) (layer F.Cu) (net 8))
 (segment (start 171.924034 108.725034) (end 172.908034 108.725034) (width 0.15) (layer F.Cu) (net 8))
 (segment (start 170.949 107.75) (end 171.924034 108.725034) (width 0.15) (layer F.Cu) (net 8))
 (segment (start 170.949 107.2) (end 170.949 107.75) (width 0.15) (layer F.Cu) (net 8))
 (segment (start 174.1455 109.3275) (end 174.383 109.3275) (width 0.15) (layer F.Cu) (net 9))
 (segment (start 172.124023 108.425023) (end 173.243023 108.425023) (width 0.15) (layer F.Cu) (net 9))
 (segment (start 171.449 107.75) (end 172.124023 108.425023) (width 0.15) (layer F.Cu) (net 9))
 (segment (start 171.449 107.2) (end 171.449 107.75) (width 0.15) (layer F.Cu) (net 9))
 (segment (start 173.243023 108.425023) (end 174.1455 109.3275) (width 0.15) (layer F.Cu) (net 9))
 (segment (start 174.1455 108.6925) (end 174.383 108.6925) (width 0.15) (layer F.Cu) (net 10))
 (segment (start 173.578011 108.125011) (end 174.1455 108.6925) (width 0.15) (layer F.Cu) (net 10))
 (segment (start 171.949 107.2) (end 171.949 107.75) (width 0.15) (layer F.Cu) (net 10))
 (segment (start 172.324011 108.125011) (end 173.578011 108.125011) (width 0.15) (layer F.Cu) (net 10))
 (segment (start 171.949 107.75) (end 172.324011 108.125011) (width 0.15) (layer F.Cu) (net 10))
 (segment (start 174.1455 108.0575) (end 174.383 108.0575) (width 0.15) (layer F.Cu) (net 11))
 (segment (start 172.449 107.75) (end 172.524001 107.825001) (width 0.15) (layer F.Cu) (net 11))
 (segment (start 173.913001 107.825001) (end 174.1455 108.0575) (width 0.15) (layer F.Cu) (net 11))
 (segment (start 172.524001 107.825001) (end 173.913001 107.825001) (width 0.15) (layer F.Cu) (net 11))
 (segment (start 172.449 107.2) (end 172.449 107.75) (width 0.15) (layer F.Cu) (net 11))
 (segment (start 174.1605 107.2) (end 174.383 107.4225) (width 0.15) (layer F.Cu) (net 12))
 (segment (start 172.949 107.2) (end 174.1605 107.2) (width 0.15) (layer F.Cu) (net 12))
 (segment (start 173.699 106.45) (end 174.0455 106.45) (width 0.15) (layer F.Cu) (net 13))
 (segment (start 174.0455 106.45) (end 174.383 106.7875) (width 0.15) (layer F.Cu) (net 13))
 (segment (start 174.1805 105.95) (end 174.383 106.1525) (width 0.15) (layer F.Cu) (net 14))
 (segment (start 173.699 105.95) (end 174.1805 105.95) (width 0.15) (layer F.Cu) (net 14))
 (segment (start 174.3155 105.45) (end 174.383 105.5175) (width 0.15) (layer F.Cu) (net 15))
 (segment (start 173.699 105.45) (end 174.3155 105.45) (width 0.15) (layer F.Cu) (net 15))
 (segment (start 174.3155 104.95) (end 174.383 104.8825) (width 0.15) (layer F.Cu) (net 16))
 (segment (start 173.699 104.95) (end 174.3155 104.95) (width 0.15) (layer F.Cu) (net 16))
 (segment (start 174.1805 104.45) (end 174.383 104.2475) (width 0.15) (layer F.Cu) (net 17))
 (segment (start 173.699 104.45) (end 174.1805 104.45) (width 0.15) (layer F.Cu) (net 17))
 (segment (start 173.699 103.95) (end 174.0455 103.95) (width 0.15) (layer F.Cu) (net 18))
 (segment (start 174.0455 103.95) (end 174.383 103.6125) (width 0.15) (layer F.Cu) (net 18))
 (segment (start 174.1605 103.2) (end 174.383 102.9775) (width 0.15) (layer F.Cu) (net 19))
 (segment (start 172.949 103.2) (end 174.1605 103.2) (width 0.15) (layer F.Cu) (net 19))
 (segment (start 174.1455 102.3425) (end 174.383 102.3425) (width 0.15) (layer F.Cu) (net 20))
 (segment (start 173.943967 102.544033) (end 174.1455 102.3425) (width 0.15) (layer F.Cu) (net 20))
 (segment (start 172.554967 102.544033) (end 173.943967 102.544033) (width 0.15) (layer F.Cu) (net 20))
 (segment (start 172.449 102.65) (end 172.554967 102.544033) (width 0.15) (layer F.Cu) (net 20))
 (segment (start 172.449 103.2) (end 172.449 102.65) (width 0.15) (layer F.Cu) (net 20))
 (segment (start 174.1455 101.7075) (end 174.383 101.7075) (width 0.15) (layer F.Cu) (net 21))
 (segment (start 173.608978 102.244022) (end 174.1455 101.7075) (width 0.15) (layer F.Cu) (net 21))
 (segment (start 172.354978 102.244022) (end 173.608978 102.244022) (width 0.15) (layer F.Cu) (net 21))
 (segment (start 171.949 102.65) (end 172.354978 102.244022) (width 0.15) (layer F.Cu) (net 21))
 (segment (start 171.949 103.2) (end 171.949 102.65) (width 0.15) (layer F.Cu) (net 21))
 (segment (start 174.1455 101.0725) (end 174.383 101.0725) (width 0.15) (layer F.Cu) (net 22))
 (segment (start 173.273989 101.944011) (end 174.1455 101.0725) (width 0.15) (layer F.Cu) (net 22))
 (segment (start 171.449 103.2) (end 171.449 102.65) (width 0.15) (layer F.Cu) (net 22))
 (segment (start 172.154989 101.944011) (end 173.273989 101.944011) (width 0.15) (layer F.Cu) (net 22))
 (segment (start 171.449 102.65) (end 172.154989 101.944011) (width 0.15) (layer F.Cu) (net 22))
 (segment (start 173.096 101.644) (end 174.3025 100.4375) (width 0.15) (layer F.Cu) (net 1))
 (segment (start 174.3025 100.4375) (end 174.383 100.4375) (width 0.15) (layer F.Cu) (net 1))
 (segment (start 171.955 101.644) (end 173.096 101.644) (width 0.15) (layer F.Cu) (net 1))
 (segment (start 170.949 103.2) (end 170.949 102.65) (width 0.15) (layer F.Cu) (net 1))
 (segment (start 170.949 102.65) (end 171.955 101.644) (width 0.15) (layer F.Cu) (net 1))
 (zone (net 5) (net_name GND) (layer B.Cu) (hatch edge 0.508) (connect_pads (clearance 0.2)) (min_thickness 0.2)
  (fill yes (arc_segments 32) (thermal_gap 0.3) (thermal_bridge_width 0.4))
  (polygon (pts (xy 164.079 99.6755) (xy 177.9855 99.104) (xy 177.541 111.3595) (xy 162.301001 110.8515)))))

